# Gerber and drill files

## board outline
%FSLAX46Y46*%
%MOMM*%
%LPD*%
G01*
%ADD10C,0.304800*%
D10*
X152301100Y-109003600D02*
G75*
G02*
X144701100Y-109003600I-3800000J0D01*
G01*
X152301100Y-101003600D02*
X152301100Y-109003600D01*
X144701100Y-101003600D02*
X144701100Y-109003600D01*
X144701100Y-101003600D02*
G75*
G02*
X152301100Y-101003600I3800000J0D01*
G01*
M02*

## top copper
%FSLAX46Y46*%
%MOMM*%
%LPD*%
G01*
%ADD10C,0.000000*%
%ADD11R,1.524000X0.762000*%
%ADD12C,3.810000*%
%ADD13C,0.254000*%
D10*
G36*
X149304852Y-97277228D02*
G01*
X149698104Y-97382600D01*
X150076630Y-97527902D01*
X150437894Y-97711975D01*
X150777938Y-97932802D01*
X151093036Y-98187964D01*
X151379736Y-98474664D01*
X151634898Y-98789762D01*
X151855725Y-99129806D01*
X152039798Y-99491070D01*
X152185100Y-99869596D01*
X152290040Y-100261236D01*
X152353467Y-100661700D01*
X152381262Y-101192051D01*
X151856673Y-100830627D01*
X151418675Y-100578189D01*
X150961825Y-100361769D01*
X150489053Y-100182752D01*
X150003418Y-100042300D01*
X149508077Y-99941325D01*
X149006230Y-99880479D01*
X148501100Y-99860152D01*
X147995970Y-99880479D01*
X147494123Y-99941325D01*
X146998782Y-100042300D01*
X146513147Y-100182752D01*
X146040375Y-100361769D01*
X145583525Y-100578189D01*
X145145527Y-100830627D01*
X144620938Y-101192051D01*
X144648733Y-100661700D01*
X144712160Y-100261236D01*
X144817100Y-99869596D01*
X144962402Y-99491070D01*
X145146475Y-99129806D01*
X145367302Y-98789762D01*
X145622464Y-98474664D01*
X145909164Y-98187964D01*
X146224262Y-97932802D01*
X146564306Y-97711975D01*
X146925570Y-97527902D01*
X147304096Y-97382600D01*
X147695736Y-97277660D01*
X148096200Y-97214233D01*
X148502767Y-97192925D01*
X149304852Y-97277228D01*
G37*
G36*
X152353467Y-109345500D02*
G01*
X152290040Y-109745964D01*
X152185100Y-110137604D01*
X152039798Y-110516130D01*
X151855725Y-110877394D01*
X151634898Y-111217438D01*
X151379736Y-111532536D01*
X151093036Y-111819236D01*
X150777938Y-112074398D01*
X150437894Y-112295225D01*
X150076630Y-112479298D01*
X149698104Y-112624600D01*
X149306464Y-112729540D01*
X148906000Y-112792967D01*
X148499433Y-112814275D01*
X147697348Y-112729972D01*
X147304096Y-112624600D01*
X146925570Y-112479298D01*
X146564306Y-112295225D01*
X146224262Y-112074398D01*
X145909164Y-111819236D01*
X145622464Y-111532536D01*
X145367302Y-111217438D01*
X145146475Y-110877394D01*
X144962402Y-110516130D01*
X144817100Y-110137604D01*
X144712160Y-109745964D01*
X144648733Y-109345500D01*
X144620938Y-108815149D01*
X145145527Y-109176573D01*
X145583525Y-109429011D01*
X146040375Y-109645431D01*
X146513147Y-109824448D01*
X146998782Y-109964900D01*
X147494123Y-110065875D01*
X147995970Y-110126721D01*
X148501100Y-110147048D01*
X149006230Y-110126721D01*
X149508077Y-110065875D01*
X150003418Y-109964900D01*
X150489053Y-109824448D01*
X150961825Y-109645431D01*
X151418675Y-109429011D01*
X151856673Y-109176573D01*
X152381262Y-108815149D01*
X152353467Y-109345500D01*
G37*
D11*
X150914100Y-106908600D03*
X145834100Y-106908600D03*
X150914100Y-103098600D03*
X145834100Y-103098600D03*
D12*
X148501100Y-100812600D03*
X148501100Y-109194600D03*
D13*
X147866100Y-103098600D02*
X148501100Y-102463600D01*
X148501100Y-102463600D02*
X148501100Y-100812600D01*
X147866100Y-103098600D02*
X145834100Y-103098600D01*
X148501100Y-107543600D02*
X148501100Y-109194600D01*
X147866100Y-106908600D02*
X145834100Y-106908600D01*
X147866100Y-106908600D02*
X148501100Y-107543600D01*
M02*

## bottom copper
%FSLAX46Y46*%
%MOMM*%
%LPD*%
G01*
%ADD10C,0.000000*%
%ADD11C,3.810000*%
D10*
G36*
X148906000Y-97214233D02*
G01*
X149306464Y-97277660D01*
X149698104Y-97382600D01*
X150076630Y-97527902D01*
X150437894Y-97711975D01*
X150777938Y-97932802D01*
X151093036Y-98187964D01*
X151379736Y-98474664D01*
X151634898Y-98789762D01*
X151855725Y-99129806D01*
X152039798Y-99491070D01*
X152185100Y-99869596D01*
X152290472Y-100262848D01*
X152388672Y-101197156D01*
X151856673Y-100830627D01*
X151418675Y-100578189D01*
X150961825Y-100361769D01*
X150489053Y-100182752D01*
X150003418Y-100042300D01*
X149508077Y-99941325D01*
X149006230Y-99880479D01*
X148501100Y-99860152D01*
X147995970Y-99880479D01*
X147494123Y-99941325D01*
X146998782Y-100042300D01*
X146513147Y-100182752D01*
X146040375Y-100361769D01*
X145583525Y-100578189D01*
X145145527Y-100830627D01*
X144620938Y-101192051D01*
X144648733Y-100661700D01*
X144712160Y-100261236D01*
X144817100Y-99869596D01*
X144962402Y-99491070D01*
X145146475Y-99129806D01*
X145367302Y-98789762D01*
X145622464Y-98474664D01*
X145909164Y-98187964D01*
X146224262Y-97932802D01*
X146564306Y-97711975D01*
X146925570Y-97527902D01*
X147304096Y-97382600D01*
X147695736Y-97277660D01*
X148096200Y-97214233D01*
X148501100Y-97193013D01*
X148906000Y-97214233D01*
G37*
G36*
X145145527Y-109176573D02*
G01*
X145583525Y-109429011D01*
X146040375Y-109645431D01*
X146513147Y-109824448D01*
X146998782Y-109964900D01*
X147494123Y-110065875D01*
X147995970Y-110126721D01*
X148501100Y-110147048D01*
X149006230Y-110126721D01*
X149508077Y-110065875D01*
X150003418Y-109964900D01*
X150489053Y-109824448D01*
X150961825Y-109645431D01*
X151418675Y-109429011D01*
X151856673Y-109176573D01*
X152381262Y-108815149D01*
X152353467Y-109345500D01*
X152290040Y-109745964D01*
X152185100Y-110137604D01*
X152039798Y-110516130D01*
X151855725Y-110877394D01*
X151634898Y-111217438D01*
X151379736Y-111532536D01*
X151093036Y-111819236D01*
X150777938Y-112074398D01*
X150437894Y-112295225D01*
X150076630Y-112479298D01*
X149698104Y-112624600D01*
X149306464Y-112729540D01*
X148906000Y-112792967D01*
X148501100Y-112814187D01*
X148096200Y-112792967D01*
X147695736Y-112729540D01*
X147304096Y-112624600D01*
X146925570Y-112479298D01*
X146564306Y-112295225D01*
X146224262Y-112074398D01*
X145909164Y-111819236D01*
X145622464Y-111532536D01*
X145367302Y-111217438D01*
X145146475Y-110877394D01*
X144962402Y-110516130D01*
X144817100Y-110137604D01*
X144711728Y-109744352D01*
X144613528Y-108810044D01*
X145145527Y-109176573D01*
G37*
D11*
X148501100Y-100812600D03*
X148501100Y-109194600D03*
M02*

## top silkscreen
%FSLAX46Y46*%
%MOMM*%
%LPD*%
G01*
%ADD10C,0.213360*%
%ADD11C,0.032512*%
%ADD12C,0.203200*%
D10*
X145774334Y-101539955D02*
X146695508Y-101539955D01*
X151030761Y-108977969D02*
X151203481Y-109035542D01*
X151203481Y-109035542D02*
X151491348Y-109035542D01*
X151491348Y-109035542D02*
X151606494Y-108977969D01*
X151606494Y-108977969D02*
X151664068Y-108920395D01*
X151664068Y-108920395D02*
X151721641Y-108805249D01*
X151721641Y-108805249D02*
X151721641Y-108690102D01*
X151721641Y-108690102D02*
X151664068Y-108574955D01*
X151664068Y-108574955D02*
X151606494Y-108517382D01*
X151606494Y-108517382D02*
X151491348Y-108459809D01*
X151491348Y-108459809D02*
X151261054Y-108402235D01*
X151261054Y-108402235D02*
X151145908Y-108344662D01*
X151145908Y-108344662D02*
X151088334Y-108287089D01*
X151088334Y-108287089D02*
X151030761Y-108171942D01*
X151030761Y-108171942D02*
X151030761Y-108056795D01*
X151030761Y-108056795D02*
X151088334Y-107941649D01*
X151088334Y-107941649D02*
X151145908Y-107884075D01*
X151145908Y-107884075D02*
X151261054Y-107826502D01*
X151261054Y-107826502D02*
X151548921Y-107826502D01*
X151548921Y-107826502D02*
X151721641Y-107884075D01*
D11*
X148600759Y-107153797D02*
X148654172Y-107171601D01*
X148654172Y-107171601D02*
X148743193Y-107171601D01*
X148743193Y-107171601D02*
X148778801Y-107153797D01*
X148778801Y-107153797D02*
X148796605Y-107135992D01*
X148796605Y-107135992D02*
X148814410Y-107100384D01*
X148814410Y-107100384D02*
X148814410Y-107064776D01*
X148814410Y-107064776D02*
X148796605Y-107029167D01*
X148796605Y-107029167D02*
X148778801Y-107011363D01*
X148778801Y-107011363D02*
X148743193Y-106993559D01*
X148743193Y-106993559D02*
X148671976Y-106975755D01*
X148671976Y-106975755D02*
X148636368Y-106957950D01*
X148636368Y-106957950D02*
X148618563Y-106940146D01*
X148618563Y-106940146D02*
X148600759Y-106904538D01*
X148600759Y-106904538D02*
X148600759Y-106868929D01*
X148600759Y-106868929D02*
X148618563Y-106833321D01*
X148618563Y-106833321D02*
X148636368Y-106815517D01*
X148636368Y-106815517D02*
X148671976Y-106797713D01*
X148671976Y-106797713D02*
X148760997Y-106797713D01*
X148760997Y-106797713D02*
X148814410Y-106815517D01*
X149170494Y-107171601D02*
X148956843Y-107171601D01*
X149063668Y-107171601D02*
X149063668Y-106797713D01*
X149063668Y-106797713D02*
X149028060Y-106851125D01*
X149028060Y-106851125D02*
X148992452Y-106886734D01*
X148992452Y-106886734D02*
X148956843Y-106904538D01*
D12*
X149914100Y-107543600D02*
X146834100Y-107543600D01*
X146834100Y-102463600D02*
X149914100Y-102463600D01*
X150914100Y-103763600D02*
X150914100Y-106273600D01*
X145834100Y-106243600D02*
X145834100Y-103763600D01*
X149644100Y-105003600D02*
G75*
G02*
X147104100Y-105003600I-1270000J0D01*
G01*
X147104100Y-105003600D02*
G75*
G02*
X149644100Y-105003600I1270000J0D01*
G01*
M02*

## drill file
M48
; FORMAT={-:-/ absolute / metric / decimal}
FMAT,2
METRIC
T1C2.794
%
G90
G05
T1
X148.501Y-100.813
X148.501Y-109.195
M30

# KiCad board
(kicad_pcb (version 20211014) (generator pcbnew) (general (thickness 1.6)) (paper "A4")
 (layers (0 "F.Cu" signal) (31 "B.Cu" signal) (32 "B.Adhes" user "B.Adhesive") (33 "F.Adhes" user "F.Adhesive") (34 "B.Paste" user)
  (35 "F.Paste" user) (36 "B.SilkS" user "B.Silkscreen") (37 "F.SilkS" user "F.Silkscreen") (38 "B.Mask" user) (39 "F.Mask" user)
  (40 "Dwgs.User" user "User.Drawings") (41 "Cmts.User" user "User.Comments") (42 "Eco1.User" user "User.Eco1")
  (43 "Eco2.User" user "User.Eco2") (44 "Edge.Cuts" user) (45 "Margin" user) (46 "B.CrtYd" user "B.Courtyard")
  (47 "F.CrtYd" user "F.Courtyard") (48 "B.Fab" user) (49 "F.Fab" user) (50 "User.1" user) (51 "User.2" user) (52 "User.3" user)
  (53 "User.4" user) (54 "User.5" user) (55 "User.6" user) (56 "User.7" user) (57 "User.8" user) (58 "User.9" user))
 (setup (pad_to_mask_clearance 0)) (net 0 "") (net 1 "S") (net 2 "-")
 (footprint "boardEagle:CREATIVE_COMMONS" (layer "F.Cu") (at 119.2911 121.5136)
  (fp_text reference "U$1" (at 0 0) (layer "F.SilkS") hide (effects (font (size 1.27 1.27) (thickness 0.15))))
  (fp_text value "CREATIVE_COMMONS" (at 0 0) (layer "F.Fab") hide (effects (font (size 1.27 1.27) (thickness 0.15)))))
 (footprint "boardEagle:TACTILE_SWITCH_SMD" (layer "F.Cu") (at 148.3741 105.0036 180)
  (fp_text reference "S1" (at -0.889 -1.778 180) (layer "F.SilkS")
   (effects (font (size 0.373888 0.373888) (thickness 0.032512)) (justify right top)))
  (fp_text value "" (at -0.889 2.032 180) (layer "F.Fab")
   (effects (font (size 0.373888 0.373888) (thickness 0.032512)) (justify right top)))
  (fp_line (start -1.54 -2.54) (end 1.54 -2.54) (layer "F.SilkS") (width 0.2032))
  (fp_line (start 1.54 2.54) (end -1.54 2.54) (layer "F.SilkS") (width 0.2032))
  (fp_line (start -2.54 1.24) (end -2.54 -1.27) (layer "F.SilkS") (width 0.2032))
  (fp_line (start 2.54 -1.24) (end 2.54 1.24) (layer "F.SilkS") (width 0.2032))
  (fp_circle (center 0 0) (end 1.27 0) (layer "F.SilkS") (width 0.2032) (fill none))
  (pad "1" smd rect (at -2.54 -1.905 270) (size 0.762 1.524) (layers "F.Cu" "F.Paste" "F.Mask") (solder_mask_margin 0.1016))
  (pad "2" smd rect (at 2.54 -1.905 270) (size 0.762 1.524) (layers "F.Cu" "F.Paste" "F.Mask") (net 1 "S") (solder_mask_margin 0.1016))
  (pad "3" smd rect (at -2.54 1.905 270) (size 0.762 1.524) (layers "F.Cu" "F.Paste" "F.Mask") (solder_mask_margin 0.1016))
  (pad "4" smd rect (at 2.54 1.905 270) (size 0.762 1.524) (layers "F.Cu" "F.Paste" "F.Mask") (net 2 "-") (solder_mask_margin 0.1016)))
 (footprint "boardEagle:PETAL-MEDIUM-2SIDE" (layer "F.Cu") (at 148.5011 101.0666 180)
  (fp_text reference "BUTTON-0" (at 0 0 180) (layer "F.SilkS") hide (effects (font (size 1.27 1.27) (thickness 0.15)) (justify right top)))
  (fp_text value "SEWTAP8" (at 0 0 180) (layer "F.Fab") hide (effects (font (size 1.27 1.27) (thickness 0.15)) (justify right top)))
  (fp_poly
   (pts (xy 3.852367 0.4049) (xy 3.78894 0.805364) (xy 3.684 1.197004) (xy 3.538698 1.57553) (xy 3.354625 1.936794) (xy 3.133798 2.276838)
    (xy 2.878636 2.591936) (xy 2.591936 2.878636) (xy 2.276838 3.133798) (xy 1.936794 3.354625) (xy 1.57553 3.538698) (xy 1.197004 3.684)
    (xy 0.805364 3.78894) (xy 0.4049 3.852367) (xy -0.001667 3.873675) (xy -0.803752 3.789372) (xy -1.197004 3.684) (xy -1.57553 3.538698)
    (xy -1.936794 3.354625) (xy -2.276838 3.133798) (xy -2.591936 2.878636) (xy -2.878636 2.591936) (xy -3.133798 2.276838)
    (xy -3.354625 1.936794) (xy -3.538698 1.57553) (xy -3.684 1.197004) (xy -3.78894 0.805364) (xy -3.852367 0.4049)
    (xy -3.880162 -0.125451) (xy -3.355573 0.235973) (xy -2.917575 0.488411) (xy -2.460725 0.704831) (xy -1.987953 0.883848)
    (xy -1.502318 1.0243) (xy -1.006977 1.125275) (xy -0.50513 1.186121) (xy 0 1.206448) (xy 0.50513 1.186121) (xy 1.006977 1.125275)
    (xy 1.502318 1.0243) (xy 1.987953 0.883848) (xy 2.460725 0.704831) (xy 2.917575 0.488411) (xy 3.355573 0.235973) (xy 3.880162 -0.125451))
   (layer "F.Cu") (width 0) (fill solid))
  (fp_poly
   (pts (xy -3.355573 0.235973) (xy -2.917575 0.488411) (xy -2.460725 0.704831) (xy -1.987953 0.883848) (xy -1.502318 1.0243)
    (xy -1.006977 1.125275) (xy -0.50513 1.186121) (xy 0 1.206448) (xy 0.50513 1.186121) (xy 1.006977 1.125275) (xy 1.502318 1.0243)
    (xy 1.987953 0.883848) (xy 2.460725 0.704831) (xy 2.917575 0.488411) (xy 3.355573 0.235973) (xy 3.880162 -0.125451) (xy 3.852367 0.4049)
    (xy 3.78894 0.805364) (xy 3.684 1.197004) (xy 3.538698 1.57553) (xy 3.354625 1.936794) (xy 3.133798 2.276838) (xy 2.878636 2.591936)
    (xy 2.591936 2.878636) (xy 2.276838 3.133798) (xy 1.936794 3.354625) (xy 1.57553 3.538698) (xy 1.197004 3.684) (xy 0.805364 3.78894)
    (xy 0.4049 3.852367) (xy 0 3.873587) (xy -0.4049 3.852367) (xy -0.805364 3.78894) (xy -1.197004 3.684) (xy -1.57553 3.538698)
    (xy -1.936794 3.354625) (xy -2.276838 3.133798) (xy -2.591936 2.878636) (xy -2.878636 2.591936) (xy -3.133798 2.276838)
    (xy -3.354625 1.936794) (xy -3.538698 1.57553) (xy -3.684 1.197004) (xy -3.789372 0.803752) (xy -3.887572 -0.130556))
   (layer "B.Cu") (width 0) (fill solid))
  (pad "1" thru_hole circle (at 0 0.254 180) (size 3.81 3.81) (drill 2.794) (layers *.Cu *.Mask) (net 2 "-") (solder_mask_margin 0.1016)))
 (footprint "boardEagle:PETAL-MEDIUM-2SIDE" (layer "F.Cu") (at 148.5011 108.9406)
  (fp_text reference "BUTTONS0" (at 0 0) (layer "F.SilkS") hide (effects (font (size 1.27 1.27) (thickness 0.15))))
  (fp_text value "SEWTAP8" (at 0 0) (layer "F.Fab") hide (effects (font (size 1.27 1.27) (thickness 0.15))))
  (fp_poly
   (pts (xy 3.852367 0.4049) (xy 3.78894 0.805364) (xy 3.684 1.197004) (xy 3.538698 1.57553) (xy 3.354625 1.936794) (xy 3.133798 2.276838)
    (xy 2.878636 2.591936) (xy 2.591936 2.878636) (xy 2.276838 3.133798) (xy 1.936794 3.354625) (xy 1.57553 3.538698) (xy 1.197004 3.684)
    (xy 0.805364 3.78894) (xy 0.4049 3.852367) (xy -0.001667 3.873675) (xy -0.803752 3.789372) (xy -1.197004 3.684) (xy -1.57553 3.538698)
    (xy -1.936794 3.354625) (xy -2.276838 3.133798) (xy -2.591936 2.878636) (xy -2.878636 2.591936) (xy -3.133798 2.276838)
    (xy -3.354625 1.936794) (xy -3.538698 1.57553) (xy -3.684 1.197004) (xy -3.78894 0.805364) (xy -3.852367 0.4049)
    (xy -3.880162 -0.125451) (xy -3.355573 0.235973) (xy -2.917575 0.488411) (xy -2.460725 0.704831) (xy -1.987953 0.883848)
    (xy -1.502318 1.0243) (xy -1.006977 1.125275) (xy -0.50513 1.186121) (xy 0 1.206448) (xy 0.50513 1.186121) (xy 1.006977 1.125275)
    (xy 1.502318 1.0243) (xy 1.987953 0.883848) (xy 2.460725 0.704831) (xy 2.917575 0.488411) (xy 3.355573 0.235973) (xy 3.880162 -0.125451))
   (layer "F.Cu") (width 0) (fill solid))
  (fp_poly
   (pts (xy -3.355573 0.235973) (xy -2.917575 0.488411) (xy -2.460725 0.704831) (xy -1.987953 0.883848) (xy -1.502318 1.0243)
    (xy -1.006977 1.125275) (xy -0.50513 1.186121) (xy 0 1.206448) (xy 0.50513 1.186121) (xy 1.006977 1.125275) (xy 1.502318 1.0243)
    (xy 1.987953 0.883848) (xy 2.460725 0.704831) (xy 2.917575 0.488411) (xy 3.355573 0.235973) (xy 3.880162 -0.125451) (xy 3.852367 0.4049)
    (xy 3.78894 0.805364) (xy 3.684 1.197004) (xy 3.538698 1.57553) (xy 3.354625 1.936794) (xy 3.133798 2.276838) (xy 2.878636 2.591936)
    (xy 2.591936 2.878636) (xy 2.276838 3.133798) (xy 1.936794 3.354625) (xy 1.57553 3.538698) (xy 1.197004 3.684) (xy 0.805364 3.78894)
    (xy 0.4049 3.852367) (xy 0 3.873587) (xy -0.4049 3.852367) (xy -0.805364 3.78894) (xy -1.197004 3.684) (xy -1.57553 3.538698)
    (xy -1.936794 3.354625) (xy -2.276838 3.133798) (xy -2.591936 2.878636) (xy -2.878636 2.591936) (xy -3.133798 2.276838)
    (xy -3.354625 1.936794) (xy -3.538698 1.57553) (xy -3.684 1.197004) (xy -3.789372 0.803752) (xy -3.887572 -0.130556))
   (layer "B.Cu") (width 0) (fill solid))
  (pad "1" thru_hole circle (at 0 0.254) (size 3.81 3.81) (drill 2.794) (layers *.Cu *.Mask) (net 1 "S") (solder_mask_margin 0.1016)))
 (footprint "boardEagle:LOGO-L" (layer "B.Cu") (at 148.5011 105.0036 180)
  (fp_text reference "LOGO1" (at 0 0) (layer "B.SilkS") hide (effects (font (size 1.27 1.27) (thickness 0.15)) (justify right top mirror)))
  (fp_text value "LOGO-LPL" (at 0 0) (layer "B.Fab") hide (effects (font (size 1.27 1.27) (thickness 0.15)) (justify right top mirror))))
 (gr_arc (start 152.3011 109.0036) (mid 148.5011 112.8036) (end 144.7011 109.0036) (layer "Edge.Cuts") (width 0.3048))
 (gr_line (start 152.3011 101.0036) (end 152.3011 109.0036) (layer "Edge.Cuts") (width 0.3048))
 (gr_line (start 144.7011 101.0036) (end 144.7011 109.0036) (layer "Edge.Cuts") (width 0.3048))
 (gr_arc (start 144.7011 101.0036) (mid 148.5011 97.2036) (end 152.3011 101.0036) (layer "Edge.Cuts") (width 0.3048))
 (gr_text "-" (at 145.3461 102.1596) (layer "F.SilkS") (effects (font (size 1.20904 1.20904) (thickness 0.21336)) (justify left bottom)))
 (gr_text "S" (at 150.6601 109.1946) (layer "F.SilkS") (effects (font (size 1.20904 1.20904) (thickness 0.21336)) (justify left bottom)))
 (segment (start 147.8661 103.0986) (end 148.5011 102.4636) (width 0.254) (layer "F.Cu") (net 2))
 (segment (start 148.5011 102.4636) (end 148.5011 100.8126) (width 0.254) (layer "F.Cu") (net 2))
 (segment (start 147.8661 103.0986) (end 145.8341 103.0986) (width 0.254) (layer "F.Cu") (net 2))
 (segment (start 148.5011 107.5436) (end 148.5011 109.1946) (width 0.254) (layer "F.Cu") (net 1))
 (segment (start 147.8661 106.9086) (end 145.8341 106.9086) (width 0.254) (layer "F.Cu") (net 1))
 (segment (start 147.8661 106.9086) (end 148.5011 107.5436) (width 0.254) (layer "F.Cu") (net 1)))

